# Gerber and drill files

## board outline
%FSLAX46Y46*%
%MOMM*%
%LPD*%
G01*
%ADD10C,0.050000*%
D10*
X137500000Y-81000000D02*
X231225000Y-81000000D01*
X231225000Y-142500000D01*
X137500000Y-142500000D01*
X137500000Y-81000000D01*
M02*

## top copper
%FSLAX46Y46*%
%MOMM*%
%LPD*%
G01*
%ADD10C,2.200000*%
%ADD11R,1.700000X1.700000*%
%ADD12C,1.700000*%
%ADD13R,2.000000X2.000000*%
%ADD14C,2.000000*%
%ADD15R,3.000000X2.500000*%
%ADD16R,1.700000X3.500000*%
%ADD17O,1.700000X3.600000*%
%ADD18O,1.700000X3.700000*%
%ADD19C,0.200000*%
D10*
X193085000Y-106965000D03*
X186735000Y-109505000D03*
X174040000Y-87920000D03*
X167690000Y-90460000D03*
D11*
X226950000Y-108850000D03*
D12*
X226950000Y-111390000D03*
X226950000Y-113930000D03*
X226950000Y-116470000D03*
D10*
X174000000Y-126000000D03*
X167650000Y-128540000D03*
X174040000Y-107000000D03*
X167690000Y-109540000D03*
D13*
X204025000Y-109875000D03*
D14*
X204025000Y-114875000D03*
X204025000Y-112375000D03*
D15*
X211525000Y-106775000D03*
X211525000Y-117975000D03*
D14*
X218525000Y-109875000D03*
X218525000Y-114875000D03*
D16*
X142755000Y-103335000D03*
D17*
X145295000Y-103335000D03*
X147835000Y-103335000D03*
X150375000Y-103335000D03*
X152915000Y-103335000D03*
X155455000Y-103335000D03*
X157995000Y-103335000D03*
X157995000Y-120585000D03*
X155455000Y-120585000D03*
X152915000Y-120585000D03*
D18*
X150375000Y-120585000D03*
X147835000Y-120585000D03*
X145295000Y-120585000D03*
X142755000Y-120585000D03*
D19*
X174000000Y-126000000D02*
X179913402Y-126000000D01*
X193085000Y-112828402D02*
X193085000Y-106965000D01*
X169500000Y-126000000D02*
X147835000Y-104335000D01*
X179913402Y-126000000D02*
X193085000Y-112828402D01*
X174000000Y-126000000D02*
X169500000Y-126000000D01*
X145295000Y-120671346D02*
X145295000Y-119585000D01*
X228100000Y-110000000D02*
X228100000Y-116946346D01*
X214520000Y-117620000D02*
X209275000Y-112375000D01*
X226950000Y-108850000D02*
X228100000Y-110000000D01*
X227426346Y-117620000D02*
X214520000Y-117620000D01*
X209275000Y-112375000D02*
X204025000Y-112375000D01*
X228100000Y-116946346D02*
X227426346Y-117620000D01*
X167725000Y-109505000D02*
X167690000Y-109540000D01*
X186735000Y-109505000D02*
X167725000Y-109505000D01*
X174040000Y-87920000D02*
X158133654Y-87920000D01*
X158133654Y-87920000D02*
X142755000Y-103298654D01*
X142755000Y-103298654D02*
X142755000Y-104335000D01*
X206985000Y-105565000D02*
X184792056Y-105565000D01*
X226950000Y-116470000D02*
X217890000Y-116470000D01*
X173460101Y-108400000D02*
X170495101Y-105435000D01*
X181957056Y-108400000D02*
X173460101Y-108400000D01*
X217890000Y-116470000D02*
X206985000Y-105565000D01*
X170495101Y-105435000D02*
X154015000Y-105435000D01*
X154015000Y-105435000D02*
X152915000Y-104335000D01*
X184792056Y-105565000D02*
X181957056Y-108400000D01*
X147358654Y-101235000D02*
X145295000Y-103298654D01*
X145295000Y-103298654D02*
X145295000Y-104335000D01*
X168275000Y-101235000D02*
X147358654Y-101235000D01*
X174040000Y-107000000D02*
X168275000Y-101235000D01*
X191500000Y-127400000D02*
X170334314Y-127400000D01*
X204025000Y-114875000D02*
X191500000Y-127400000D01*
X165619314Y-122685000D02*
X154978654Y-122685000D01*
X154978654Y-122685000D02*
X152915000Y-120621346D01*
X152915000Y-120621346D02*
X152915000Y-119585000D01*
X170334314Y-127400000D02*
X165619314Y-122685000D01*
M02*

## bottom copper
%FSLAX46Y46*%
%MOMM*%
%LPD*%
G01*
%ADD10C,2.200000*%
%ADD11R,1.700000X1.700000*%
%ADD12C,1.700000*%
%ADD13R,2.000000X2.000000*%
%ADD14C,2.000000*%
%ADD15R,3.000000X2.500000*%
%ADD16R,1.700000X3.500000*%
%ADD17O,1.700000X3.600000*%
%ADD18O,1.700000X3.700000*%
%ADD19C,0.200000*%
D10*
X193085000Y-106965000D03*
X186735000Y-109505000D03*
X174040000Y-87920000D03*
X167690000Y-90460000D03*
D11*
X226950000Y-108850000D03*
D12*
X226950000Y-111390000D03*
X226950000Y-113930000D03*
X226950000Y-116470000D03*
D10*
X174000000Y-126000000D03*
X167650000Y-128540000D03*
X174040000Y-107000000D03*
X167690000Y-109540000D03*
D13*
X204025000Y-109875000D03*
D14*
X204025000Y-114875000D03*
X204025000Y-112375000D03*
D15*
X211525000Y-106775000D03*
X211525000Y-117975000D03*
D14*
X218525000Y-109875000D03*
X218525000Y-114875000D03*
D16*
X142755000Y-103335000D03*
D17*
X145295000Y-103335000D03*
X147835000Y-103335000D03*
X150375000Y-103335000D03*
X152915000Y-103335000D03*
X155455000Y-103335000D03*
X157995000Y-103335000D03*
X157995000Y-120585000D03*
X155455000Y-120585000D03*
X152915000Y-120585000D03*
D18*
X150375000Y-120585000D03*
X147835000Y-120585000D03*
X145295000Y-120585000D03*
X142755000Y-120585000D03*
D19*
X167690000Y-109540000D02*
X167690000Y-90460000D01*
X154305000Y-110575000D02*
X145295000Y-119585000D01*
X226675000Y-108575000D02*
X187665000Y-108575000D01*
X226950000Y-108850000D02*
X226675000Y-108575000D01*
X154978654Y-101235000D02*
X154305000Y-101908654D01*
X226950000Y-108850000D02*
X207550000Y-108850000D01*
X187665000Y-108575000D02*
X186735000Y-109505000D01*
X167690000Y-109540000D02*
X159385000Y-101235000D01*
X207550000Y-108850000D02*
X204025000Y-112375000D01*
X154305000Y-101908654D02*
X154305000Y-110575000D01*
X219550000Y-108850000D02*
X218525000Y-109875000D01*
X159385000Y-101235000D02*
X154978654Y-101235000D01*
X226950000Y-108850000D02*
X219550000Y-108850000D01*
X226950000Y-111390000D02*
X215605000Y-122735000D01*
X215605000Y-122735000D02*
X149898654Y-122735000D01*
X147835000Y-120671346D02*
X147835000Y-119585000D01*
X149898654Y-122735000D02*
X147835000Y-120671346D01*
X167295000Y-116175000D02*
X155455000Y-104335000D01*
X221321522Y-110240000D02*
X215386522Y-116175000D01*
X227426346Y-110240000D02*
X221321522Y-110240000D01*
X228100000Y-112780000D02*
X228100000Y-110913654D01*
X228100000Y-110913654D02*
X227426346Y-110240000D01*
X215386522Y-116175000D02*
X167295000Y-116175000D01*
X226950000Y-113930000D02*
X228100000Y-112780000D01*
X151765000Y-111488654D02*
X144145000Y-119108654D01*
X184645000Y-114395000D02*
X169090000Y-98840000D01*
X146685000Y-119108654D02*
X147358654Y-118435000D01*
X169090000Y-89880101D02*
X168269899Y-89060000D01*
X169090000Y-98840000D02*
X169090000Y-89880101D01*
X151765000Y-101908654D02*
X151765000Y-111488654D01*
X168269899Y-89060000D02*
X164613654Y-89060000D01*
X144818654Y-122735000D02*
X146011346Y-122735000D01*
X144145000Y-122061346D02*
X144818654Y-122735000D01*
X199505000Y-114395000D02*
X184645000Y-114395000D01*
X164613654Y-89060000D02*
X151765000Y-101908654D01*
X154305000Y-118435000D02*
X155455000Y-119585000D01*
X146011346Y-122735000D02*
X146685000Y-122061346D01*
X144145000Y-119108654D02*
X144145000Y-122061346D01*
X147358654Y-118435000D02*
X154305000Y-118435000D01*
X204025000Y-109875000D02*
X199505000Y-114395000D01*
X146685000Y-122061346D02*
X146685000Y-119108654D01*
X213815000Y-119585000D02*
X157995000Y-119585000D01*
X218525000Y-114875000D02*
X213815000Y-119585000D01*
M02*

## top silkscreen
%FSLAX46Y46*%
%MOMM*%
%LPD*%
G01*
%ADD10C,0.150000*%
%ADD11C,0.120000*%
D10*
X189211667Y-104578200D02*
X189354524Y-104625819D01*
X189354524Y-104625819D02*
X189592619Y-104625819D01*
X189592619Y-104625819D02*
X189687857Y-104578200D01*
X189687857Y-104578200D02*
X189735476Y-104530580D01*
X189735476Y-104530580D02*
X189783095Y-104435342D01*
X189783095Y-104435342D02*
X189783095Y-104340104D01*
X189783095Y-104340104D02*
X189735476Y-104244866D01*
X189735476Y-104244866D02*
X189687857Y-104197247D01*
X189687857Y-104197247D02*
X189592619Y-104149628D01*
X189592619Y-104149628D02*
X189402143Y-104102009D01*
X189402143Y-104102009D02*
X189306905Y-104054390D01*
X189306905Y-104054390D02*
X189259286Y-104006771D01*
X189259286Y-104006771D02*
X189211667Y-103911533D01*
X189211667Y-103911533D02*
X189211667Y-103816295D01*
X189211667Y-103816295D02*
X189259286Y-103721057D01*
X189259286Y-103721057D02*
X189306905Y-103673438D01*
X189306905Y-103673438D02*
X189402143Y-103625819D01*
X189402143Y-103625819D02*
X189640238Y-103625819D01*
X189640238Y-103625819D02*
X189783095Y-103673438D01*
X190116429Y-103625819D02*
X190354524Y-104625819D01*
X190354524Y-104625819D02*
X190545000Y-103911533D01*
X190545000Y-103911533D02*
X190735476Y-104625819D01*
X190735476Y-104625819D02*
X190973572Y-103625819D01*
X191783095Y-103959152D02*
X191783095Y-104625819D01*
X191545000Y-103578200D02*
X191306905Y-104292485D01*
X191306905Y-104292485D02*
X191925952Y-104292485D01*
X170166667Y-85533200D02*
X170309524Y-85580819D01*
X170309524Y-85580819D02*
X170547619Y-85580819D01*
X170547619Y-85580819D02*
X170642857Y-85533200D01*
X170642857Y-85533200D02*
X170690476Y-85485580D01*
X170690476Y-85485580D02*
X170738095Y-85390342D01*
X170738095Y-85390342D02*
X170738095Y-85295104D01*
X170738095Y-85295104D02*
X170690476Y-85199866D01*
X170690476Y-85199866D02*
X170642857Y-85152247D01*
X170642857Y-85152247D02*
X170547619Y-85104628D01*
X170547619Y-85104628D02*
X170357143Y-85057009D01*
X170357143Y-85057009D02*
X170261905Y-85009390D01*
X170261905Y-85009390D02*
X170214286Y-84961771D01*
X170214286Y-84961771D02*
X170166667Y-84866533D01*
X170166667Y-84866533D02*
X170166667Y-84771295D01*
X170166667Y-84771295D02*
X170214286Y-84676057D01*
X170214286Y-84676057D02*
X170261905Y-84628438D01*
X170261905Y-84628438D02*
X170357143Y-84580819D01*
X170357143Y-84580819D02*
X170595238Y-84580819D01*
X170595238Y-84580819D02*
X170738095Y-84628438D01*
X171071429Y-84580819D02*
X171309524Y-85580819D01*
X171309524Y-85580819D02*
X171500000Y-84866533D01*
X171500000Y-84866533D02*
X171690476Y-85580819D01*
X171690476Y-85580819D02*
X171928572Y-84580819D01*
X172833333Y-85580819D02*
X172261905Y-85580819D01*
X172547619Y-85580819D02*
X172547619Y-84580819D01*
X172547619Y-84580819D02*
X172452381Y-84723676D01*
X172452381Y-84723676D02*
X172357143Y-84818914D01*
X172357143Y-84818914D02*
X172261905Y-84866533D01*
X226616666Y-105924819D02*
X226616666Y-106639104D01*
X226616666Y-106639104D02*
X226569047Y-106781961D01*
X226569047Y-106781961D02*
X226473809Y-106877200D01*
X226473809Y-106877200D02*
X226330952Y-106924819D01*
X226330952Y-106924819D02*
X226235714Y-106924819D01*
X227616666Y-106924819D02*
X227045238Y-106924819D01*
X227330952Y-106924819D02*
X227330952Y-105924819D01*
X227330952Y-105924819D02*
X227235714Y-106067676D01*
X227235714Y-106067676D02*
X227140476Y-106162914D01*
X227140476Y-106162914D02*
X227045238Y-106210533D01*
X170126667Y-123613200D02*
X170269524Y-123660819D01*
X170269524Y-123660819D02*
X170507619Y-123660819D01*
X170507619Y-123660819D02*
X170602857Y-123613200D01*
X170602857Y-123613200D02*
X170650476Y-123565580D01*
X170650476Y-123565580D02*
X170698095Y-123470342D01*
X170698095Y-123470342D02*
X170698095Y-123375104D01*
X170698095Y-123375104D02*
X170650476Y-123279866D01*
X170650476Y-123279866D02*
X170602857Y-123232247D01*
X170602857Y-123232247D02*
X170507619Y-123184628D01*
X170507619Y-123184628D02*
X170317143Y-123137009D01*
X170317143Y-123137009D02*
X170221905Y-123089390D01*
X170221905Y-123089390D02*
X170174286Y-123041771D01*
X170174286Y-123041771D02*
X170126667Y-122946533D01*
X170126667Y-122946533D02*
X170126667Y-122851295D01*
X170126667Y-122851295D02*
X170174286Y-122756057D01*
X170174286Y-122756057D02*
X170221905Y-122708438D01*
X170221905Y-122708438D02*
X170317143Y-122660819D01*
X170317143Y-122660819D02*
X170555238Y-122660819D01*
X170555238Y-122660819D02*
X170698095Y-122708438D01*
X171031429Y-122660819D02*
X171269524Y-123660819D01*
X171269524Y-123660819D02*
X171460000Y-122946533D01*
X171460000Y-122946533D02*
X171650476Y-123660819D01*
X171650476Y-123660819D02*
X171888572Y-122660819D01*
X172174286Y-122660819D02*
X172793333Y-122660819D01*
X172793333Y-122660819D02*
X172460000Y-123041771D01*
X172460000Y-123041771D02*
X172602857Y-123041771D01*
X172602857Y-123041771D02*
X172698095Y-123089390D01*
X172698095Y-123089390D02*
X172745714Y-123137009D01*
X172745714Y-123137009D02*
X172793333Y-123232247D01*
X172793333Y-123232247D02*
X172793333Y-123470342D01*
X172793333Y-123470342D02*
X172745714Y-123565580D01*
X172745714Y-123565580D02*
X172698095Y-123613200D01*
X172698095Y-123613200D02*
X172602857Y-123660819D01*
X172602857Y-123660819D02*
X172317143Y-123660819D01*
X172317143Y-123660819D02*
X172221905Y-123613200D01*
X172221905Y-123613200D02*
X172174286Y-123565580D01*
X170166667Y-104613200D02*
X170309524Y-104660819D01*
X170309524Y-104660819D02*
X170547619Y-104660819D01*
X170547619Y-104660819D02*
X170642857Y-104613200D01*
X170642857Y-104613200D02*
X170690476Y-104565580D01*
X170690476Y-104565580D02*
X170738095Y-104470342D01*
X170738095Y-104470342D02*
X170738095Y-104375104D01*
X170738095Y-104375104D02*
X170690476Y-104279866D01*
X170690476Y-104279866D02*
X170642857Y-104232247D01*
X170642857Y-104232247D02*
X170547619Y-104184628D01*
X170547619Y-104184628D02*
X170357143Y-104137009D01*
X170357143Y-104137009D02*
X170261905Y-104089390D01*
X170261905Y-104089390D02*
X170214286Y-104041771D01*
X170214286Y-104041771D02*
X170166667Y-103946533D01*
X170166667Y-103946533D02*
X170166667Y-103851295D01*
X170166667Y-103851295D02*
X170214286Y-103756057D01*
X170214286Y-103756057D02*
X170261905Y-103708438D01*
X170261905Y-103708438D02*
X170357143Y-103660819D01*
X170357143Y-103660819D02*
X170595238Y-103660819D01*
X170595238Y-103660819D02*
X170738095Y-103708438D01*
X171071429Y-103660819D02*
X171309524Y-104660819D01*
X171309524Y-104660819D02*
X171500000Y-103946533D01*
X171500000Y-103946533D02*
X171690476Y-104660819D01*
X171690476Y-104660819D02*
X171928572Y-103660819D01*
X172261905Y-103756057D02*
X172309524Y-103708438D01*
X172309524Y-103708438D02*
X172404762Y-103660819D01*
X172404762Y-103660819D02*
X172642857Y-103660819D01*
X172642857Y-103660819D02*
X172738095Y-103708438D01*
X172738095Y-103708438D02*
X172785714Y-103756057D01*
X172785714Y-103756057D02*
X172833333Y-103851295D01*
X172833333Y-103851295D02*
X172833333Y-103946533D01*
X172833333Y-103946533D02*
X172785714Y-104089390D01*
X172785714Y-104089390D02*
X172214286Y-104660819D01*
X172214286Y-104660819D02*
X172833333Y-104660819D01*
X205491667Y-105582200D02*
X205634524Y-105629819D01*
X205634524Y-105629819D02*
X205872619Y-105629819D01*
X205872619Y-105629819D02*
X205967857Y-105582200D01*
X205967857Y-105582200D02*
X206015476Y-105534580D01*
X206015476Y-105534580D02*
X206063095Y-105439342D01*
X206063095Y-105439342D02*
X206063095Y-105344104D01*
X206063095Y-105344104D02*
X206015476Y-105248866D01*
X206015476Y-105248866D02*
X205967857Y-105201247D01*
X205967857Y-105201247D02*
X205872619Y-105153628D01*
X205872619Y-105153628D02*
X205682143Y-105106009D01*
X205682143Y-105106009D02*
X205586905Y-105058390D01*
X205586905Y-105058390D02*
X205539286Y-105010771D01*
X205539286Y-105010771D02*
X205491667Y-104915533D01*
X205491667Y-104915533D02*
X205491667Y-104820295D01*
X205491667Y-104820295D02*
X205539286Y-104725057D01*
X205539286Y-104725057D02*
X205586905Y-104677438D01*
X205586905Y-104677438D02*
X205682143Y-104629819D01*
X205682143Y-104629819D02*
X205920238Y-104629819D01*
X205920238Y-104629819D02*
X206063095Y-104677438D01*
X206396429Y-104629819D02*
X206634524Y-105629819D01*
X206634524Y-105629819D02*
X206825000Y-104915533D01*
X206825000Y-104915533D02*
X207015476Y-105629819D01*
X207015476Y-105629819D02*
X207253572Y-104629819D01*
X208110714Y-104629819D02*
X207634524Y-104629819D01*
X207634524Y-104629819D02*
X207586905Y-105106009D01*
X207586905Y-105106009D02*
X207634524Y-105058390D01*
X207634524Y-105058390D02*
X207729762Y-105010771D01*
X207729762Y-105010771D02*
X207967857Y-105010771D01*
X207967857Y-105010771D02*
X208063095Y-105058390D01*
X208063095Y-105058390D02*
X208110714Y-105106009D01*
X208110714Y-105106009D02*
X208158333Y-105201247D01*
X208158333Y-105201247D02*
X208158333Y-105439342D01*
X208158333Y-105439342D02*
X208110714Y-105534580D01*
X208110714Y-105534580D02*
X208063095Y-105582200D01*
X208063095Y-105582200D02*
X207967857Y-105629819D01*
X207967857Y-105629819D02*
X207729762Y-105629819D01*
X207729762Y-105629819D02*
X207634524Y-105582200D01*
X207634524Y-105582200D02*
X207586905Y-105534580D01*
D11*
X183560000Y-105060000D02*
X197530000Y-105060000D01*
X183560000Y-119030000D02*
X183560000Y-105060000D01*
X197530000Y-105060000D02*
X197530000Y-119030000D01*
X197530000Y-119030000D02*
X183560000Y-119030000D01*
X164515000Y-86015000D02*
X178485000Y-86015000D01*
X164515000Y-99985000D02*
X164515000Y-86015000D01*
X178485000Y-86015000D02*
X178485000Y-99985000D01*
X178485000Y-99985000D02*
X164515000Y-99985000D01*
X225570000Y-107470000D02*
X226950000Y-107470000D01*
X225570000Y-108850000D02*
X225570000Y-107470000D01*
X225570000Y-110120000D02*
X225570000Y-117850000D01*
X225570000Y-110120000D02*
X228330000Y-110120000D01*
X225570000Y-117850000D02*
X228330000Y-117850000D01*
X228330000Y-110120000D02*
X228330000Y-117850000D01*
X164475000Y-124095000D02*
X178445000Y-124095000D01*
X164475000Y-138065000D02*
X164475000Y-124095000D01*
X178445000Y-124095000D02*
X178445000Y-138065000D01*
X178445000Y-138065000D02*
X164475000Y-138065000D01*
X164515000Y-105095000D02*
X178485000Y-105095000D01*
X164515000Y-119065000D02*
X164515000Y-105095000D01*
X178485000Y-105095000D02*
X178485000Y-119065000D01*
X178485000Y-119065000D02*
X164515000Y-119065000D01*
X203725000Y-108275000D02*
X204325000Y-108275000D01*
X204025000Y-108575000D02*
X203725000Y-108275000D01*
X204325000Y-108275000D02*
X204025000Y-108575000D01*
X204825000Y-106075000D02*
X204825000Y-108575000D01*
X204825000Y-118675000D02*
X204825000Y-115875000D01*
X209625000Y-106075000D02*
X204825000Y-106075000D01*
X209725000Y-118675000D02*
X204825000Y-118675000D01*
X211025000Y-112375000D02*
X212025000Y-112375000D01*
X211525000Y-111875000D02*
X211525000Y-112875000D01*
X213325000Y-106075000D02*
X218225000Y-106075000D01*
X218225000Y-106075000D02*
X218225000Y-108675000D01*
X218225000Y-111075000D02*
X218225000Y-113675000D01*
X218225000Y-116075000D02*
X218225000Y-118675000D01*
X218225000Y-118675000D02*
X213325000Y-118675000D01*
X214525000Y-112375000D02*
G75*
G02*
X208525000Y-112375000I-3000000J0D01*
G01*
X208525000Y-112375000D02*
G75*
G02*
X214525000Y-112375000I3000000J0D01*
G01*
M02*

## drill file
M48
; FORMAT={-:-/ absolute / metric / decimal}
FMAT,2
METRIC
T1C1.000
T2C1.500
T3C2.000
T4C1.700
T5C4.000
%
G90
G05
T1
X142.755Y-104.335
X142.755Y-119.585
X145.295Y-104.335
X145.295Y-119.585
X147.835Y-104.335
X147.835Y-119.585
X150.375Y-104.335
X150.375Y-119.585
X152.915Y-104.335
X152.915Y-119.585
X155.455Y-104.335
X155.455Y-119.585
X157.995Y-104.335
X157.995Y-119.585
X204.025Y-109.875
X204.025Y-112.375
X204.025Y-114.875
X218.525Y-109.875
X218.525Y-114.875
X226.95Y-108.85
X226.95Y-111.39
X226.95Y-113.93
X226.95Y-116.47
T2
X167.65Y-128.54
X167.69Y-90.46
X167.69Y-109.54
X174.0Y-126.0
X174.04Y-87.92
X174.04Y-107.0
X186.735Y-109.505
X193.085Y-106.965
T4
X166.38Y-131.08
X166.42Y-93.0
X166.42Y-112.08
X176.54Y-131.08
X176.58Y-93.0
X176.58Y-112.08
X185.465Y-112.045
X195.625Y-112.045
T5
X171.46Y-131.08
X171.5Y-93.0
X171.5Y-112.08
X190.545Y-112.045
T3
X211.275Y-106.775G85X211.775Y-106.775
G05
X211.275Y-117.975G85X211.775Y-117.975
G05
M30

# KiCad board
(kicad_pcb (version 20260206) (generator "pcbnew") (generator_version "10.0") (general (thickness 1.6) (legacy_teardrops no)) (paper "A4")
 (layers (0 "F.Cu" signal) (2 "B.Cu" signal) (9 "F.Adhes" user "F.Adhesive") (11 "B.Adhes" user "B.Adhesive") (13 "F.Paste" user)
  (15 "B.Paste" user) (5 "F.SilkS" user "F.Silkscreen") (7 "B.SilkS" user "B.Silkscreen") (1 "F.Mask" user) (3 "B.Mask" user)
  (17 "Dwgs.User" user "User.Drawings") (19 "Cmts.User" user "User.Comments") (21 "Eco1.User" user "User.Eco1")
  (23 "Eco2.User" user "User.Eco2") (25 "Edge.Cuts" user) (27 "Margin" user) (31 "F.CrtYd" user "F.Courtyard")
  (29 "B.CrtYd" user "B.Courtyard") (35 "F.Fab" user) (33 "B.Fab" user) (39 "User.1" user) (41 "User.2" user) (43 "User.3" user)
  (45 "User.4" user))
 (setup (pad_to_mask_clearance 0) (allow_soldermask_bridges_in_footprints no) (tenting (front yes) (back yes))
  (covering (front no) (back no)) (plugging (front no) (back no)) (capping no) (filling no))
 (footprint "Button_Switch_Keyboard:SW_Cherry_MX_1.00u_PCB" (layer "F.Cu") (at 193.085 106.965)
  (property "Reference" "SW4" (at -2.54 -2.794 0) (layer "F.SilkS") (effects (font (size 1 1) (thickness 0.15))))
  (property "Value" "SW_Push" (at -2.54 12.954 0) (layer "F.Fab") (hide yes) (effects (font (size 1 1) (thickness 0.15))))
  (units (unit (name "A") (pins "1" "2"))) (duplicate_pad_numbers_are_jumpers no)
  (fp_line (start -9.525 -1.905) (end 4.445 -1.905) (stroke (width 0.12) (type solid)) (layer "F.SilkS"))
  (fp_line (start -9.525 12.065) (end -9.525 -1.905) (stroke (width 0.12) (type solid)) (layer "F.SilkS"))
  (fp_line (start 4.445 -1.905) (end 4.445 12.065) (stroke (width 0.12) (type solid)) (layer "F.SilkS"))
  (fp_line (start 4.445 12.065) (end -9.525 12.065) (stroke (width 0.12) (type solid)) (layer "F.SilkS"))
  (pad "" np_thru_hole circle (at -7.62 5.08) (size 1.7 1.7) (drill 1.7) (layers "*.Cu" "*.Mask"))
  (pad "" np_thru_hole circle (at -2.54 5.08) (size 4 4) (drill 4) (layers "*.Cu" "*.Mask"))
  (pad "" np_thru_hole circle (at 2.54 5.08) (size 1.7 1.7) (drill 1.7) (layers "*.Cu" "*.Mask"))
  (pad "1" thru_hole circle (at 0 0) (size 2.2 2.2) (drill 1.5) (layers "*.Cu" "*.Mask") (remove_unused_layers no)
   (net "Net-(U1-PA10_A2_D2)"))
  (pad "2" thru_hole circle (at -6.35 2.54) (size 2.2 2.2) (drill 1.5) (layers "*.Cu" "*.Mask") (remove_unused_layers no) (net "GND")))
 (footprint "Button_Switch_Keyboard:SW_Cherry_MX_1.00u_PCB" (layer "F.Cu") (at 174.04 87.92)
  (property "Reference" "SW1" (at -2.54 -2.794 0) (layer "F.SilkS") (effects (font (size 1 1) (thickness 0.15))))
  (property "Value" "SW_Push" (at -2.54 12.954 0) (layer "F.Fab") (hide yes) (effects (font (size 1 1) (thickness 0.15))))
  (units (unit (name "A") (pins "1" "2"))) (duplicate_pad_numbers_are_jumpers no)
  (fp_line (start -9.525 -1.905) (end 4.445 -1.905) (stroke (width 0.12) (type solid)) (layer "F.SilkS"))
  (fp_line (start -9.525 12.065) (end -9.525 -1.905) (stroke (width 0.12) (type solid)) (layer "F.SilkS"))
  (fp_line (start 4.445 -1.905) (end 4.445 12.065) (stroke (width 0.12) (type solid)) (layer "F.SilkS"))
  (fp_line (start 4.445 12.065) (end -9.525 12.065) (stroke (width 0.12) (type solid)) (layer "F.SilkS"))
  (pad "" np_thru_hole circle (at -7.62 5.08) (size 1.7 1.7) (drill 1.7) (layers "*.Cu" "*.Mask"))
  (pad "" np_thru_hole circle (at -2.54 5.08) (size 4 4) (drill 4) (layers "*.Cu" "*.Mask"))
  (pad "" np_thru_hole circle (at 2.54 5.08) (size 1.7 1.7) (drill 1.7) (layers "*.Cu" "*.Mask"))
  (pad "1" thru_hole circle (at 0 0) (size 2.2 2.2) (drill 1.5) (layers "*.Cu" "*.Mask") (remove_unused_layers no)
   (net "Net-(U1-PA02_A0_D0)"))
  (pad "2" thru_hole circle (at -6.35 2.54) (size 2.2 2.2) (drill 1.5) (layers "*.Cu" "*.Mask") (remove_unused_layers no) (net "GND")))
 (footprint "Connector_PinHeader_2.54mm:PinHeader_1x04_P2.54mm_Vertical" (layer "F.Cu") (at 226.95 108.85)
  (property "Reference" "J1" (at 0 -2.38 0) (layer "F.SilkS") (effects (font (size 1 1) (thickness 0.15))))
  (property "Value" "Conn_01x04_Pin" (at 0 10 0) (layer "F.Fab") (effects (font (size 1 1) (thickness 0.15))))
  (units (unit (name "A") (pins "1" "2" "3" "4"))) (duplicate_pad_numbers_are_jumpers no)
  (fp_line (start -1.38 -1.38) (end 0 -1.38) (stroke (width 0.12) (type solid)) (layer "F.SilkS"))
  (fp_line (start -1.38 0) (end -1.38 -1.38) (stroke (width 0.12) (type solid)) (layer "F.SilkS"))
  (fp_line (start -1.38 1.27) (end -1.38 9) (stroke (width 0.12) (type solid)) (layer "F.SilkS"))
  (fp_line (start -1.38 1.27) (end 1.38 1.27) (stroke (width 0.12) (type solid)) (layer "F.SilkS"))
  (fp_line (start -1.38 9) (end 1.38 9) (stroke (width 0.12) (type solid)) (layer "F.SilkS"))
  (fp_line (start 1.38 1.27) (end 1.38 9) (stroke (width 0.12) (type solid)) (layer "F.SilkS"))
  (pad "1" thru_hole rect (at 0 0) (size 1.7 1.7) (drill 1) (layers "*.Cu" "*.Mask") (remove_unused_layers no) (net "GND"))
  (pad "2" thru_hole circle (at 0 2.54) (size 1.7 1.7) (drill 1) (layers "*.Cu" "*.Mask") (remove_unused_layers no) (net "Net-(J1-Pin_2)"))
  (pad "3" thru_hole circle (at 0 5.08) (size 1.7 1.7) (drill 1) (layers "*.Cu" "*.Mask") (remove_unused_layers no) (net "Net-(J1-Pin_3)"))
  (pad "4" thru_hole circle (at 0 7.62) (size 1.7 1.7) (drill 1) (layers "*.Cu" "*.Mask") (remove_unused_layers no) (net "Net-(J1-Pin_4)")))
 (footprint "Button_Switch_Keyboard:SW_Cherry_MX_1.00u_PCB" (layer "F.Cu") (at 174 126)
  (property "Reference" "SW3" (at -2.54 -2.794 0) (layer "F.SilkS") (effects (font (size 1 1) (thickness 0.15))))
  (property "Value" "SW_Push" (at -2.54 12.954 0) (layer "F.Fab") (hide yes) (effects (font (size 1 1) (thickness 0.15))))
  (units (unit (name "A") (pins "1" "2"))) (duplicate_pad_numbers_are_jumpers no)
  (fp_line (start -9.525 -1.905) (end 4.445 -1.905) (stroke (width 0.12) (type solid)) (layer "F.SilkS"))
  (fp_line (start -9.525 12.065) (end -9.525 -1.905) (stroke (width 0.12) (type solid)) (layer "F.SilkS"))
  (fp_line (start 4.445 -1.905) (end 4.445 12.065) (stroke (width 0.12) (type solid)) (layer "F.SilkS"))
  (fp_line (start 4.445 12.065) (end -9.525 12.065) (stroke (width 0.12) (type solid)) (layer "F.SilkS"))
  (pad "" np_thru_hole circle (at -7.62 5.08) (size 1.7 1.7) (drill 1.7) (layers "*.Cu" "*.Mask"))
  (pad "" np_thru_hole circle (at -2.54 5.08) (size 4 4) (drill 4) (layers "*.Cu" "*.Mask"))
  (pad "" np_thru_hole circle (at 2.54 5.08) (size 1.7 1.7) (drill 1.7) (layers "*.Cu" "*.Mask"))
  (pad "1" thru_hole circle (at 0 0) (size 2.2 2.2) (drill 1.5) (layers "*.Cu" "*.Mask") (remove_unused_layers no)
   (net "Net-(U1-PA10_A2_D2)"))
  (pad "2" thru_hole circle (at -6.35 2.54) (size 2.2 2.2) (drill 1.5) (layers "*.Cu" "*.Mask") (remove_unused_layers no) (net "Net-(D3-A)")))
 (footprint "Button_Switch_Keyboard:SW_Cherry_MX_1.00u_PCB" (layer "F.Cu") (at 174.04 107)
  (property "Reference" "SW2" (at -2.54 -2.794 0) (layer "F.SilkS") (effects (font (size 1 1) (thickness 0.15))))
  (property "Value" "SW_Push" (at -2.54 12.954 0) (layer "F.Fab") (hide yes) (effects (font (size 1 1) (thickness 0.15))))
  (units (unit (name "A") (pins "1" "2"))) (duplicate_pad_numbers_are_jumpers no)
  (fp_line (start -9.525 -1.905) (end 4.445 -1.905) (stroke (width 0.12) (type solid)) (layer "F.SilkS"))
  (fp_line (start -9.525 12.065) (end -9.525 -1.905) (stroke (width 0.12) (type solid)) (layer "F.SilkS"))
  (fp_line (start 4.445 -1.905) (end 4.445 12.065) (stroke (width 0.12) (type solid)) (layer "F.SilkS"))
  (fp_line (start 4.445 12.065) (end -9.525 12.065) (stroke (width 0.12) (type solid)) (layer "F.SilkS"))
  (pad "" np_thru_hole circle (at -7.62 5.08) (size 1.7 1.7) (drill 1.7) (layers "*.Cu" "*.Mask"))
  (pad "" np_thru_hole circle (at -2.54 5.08) (size 4 4) (drill 4) (layers "*.Cu" "*.Mask"))
  (pad "" np_thru_hole circle (at 2.54 5.08) (size 1.7 1.7) (drill 1.7) (layers "*.Cu" "*.Mask"))
  (pad "1" thru_hole circle (at 0 0) (size 2.2 2.2) (drill 1.5) (layers "*.Cu" "*.Mask") (remove_unused_layers no)
   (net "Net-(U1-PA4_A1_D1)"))
  (pad "2" thru_hole circle (at -6.35 2.54) (size 2.2 2.2) (drill 1.5) (layers "*.Cu" "*.Mask") (remove_unused_layers no) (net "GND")))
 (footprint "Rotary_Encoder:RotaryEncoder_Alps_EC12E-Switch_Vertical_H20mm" (layer "F.Cu") (at 204.025 109.875)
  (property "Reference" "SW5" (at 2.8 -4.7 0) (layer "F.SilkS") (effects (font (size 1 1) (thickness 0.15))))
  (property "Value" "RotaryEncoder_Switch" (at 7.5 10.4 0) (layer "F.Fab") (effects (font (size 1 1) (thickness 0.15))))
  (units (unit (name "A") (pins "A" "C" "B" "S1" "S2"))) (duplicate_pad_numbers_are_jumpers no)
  (fp_line (start -0.3 -1.6) (end 0.3 -1.6) (stroke (width 0.12) (type solid)) (layer "F.SilkS"))
  (fp_line (start 0 -1.3) (end -0.3 -1.6) (stroke (width 0.12) (type solid)) (layer "F.SilkS"))
  (fp_line (start 0.3 -1.6) (end 0 -1.3) (stroke (width 0.12) (type solid)) (layer "F.SilkS"))
  (fp_line (start 0.8 -3.8) (end 0.8 -1.3) (stroke (width 0.12) (type solid)) (layer "F.SilkS"))
  (fp_line (start 0.8 8.8) (end 0.8 6) (stroke (width 0.12) (type solid)) (layer "F.SilkS"))
  (fp_line (start 5.6 -3.8) (end 0.8 -3.8) (stroke (width 0.12) (type solid)) (layer "F.SilkS"))
  (fp_line (start 5.7 8.8) (end 0.8 8.8) (stroke (width 0.12) (type solid)) (layer "F.SilkS"))
  (fp_line (start 7 2.5) (end 8 2.5) (stroke (width 0.12) (type solid)) (layer "F.SilkS"))
  (fp_line (start 7.5 2) (end 7.5 3) (stroke (width 0.12) (type solid)) (layer "F.SilkS"))
  (fp_line (start 9.3 -3.8) (end 14.2 -3.8) (stroke (width 0.12) (type solid)) (layer "F.SilkS"))
  (fp_line (start 14.2 -3.8) (end 14.2 -1.2) (stroke (width 0.12) (type solid)) (layer "F.SilkS"))
  (fp_line (start 14.2 1.2) (end 14.2 3.8) (stroke (width 0.12) (type solid)) (layer "F.SilkS"))
  (fp_line (start 14.2 6.2) (end 14.2 8.8) (stroke (width 0.12) (type solid)) (layer "F.SilkS"))
  (fp_line (start 14.2 8.8) (end 9.3 8.8) (stroke (width 0.12) (type solid)) (layer "F.SilkS"))
  (fp_circle (center 7.5 2.5) (end 10.5 2.5) (stroke (width 0.12) (type solid)) (fill no) (layer "F.SilkS"))
  (pad "A" thru_hole rect (at 0 0) (size 2 2) (drill 1) (layers "*.Cu" "*.Mask") (remove_unused_layers no) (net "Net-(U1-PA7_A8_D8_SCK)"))
  (pad "B" thru_hole circle (at 0 5) (size 2 2) (drill 1) (layers "*.Cu" "*.Mask") (remove_unused_layers no) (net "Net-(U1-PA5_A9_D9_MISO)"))
  (pad "C" thru_hole circle (at 0 2.5) (size 2 2) (drill 1) (layers "*.Cu" "*.Mask") (remove_unused_layers no) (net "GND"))
  (pad "MP" thru_hole rect (at 7.5 -3.1) (size 3 2.5) (drill oval 2.5 2) (layers "*.Cu" "*.Mask") (remove_unused_layers no))
  (pad "MP" thru_hole rect (at 7.5 8.1) (size 3 2.5) (drill oval 2.5 2) (layers "*.Cu" "*.Mask") (remove_unused_layers no))
  (pad "S1" thru_hole circle (at 14.5 0) (size 2 2) (drill 1) (layers "*.Cu" "*.Mask") (remove_unused_layers no) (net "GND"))
  (pad "S2" thru_hole circle (at 14.5 5) (size 2 2) (drill 1) (layers "*.Cu" "*.Mask") (remove_unused_layers no)
   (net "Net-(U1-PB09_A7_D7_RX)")))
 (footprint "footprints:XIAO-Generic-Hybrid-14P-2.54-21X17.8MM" (layer "B.Cu") (at 150.375 111.96 -90)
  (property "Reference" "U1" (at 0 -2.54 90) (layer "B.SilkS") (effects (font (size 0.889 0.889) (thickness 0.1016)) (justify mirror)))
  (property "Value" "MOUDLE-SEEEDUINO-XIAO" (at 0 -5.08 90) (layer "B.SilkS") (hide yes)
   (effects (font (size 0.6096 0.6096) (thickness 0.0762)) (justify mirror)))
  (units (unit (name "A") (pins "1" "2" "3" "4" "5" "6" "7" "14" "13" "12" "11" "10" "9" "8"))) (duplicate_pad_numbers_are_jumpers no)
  (pad "1" thru_hole rect (at -7.625 7.62 270) (size 3.5 1.7) (drill 1 (offset -1 0)) (layers "*.Cu" "*.Mask") (remove_unused_layers no)
   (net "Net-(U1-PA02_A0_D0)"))
  (pad "2" thru_hole oval (at -7.625 5.08 270) (size 3.6 1.7) (drill 1 (offset -1 0)) (layers "*.Cu" "*.Mask") (remove_unused_layers no)
   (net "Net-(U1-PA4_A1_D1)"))
  (pad "3" thru_hole oval (at -7.625 2.54 270) (size 3.6 1.7) (drill 1 (offset -1 0)) (layers "*.Cu" "*.Mask") (remove_unused_layers no)
   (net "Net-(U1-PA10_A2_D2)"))
  (pad "4" thru_hole oval (at -7.625 0 270) (size 3.6 1.7) (drill 1 (offset -1 0)) (layers "*.Cu" "*.Mask") (remove_unused_layers no)
   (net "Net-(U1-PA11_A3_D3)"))
  (pad "5" thru_hole oval (at -7.625 -2.54 270) (size 3.6 1.7) (drill 1 (offset -1 0)) (layers "*.Cu" "*.Mask") (remove_unused_layers no)
   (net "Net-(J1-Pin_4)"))
  (pad "6" thru_hole oval (at -7.625 -5.08 90) (size 3.6 1.7) (drill 1 (offset 1 0)) (layers "*.Cu" "*.Mask") (remove_unused_layers no)
   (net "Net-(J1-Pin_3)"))
  (pad "7" thru_hole oval (at -7.625 -7.62 270) (size 3.6 1.7) (drill 1 (offset -1 0)) (layers "*.Cu" "*.Mask") (remove_unused_layers no)
   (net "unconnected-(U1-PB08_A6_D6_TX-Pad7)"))
  (pad "8" thru_hole oval (at 7.625 -7.62 270) (size 3.6 1.7) (drill 1 (offset 1 0)) (layers "*.Cu" "*.Mask") (remove_unused_layers no)
   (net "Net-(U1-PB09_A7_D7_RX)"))
  (pad "9" thru_hole oval (at 7.625 -5.08 270) (size 3.6 1.7) (drill 1 (offset 1 0)) (layers "*.Cu" "*.Mask") (remove_unused_layers no)
   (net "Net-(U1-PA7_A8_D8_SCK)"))
  (pad "10" thru_hole oval (at 7.625 -2.54 270) (size 3.6 1.7) (drill 1 (offset 1 0)) (layers "*.Cu" "*.Mask") (remove_unused_layers no)
   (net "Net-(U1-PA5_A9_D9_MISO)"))
  (pad "11" thru_hole oval (at 7.625 0 270) (size 3.7 1.7) (drill 1 (offset 1 0)) (layers "*.Cu" "*.Mask") (remove_unused_layers no)
   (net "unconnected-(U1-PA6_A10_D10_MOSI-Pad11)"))
  (pad "12" thru_hole oval (at 7.625 2.54 270) (size 3.7 1.7) (drill 1 (offset 1 0)) (layers "*.Cu" "*.Mask") (remove_unused_layers no)
   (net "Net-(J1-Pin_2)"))
  (pad "13" thru_hole oval (at 7.625 5.08 270) (size 3.7 1.7) (drill 1 (offset 1 0)) (layers "*.Cu" "*.Mask") (remove_unused_layers no)
   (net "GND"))
  (pad "14" thru_hole oval (at 7.625 7.62 270) (size 3.7 1.7) (drill 1 (offset 1 0)) (layers "*.Cu" "*.Mask") (remove_unused_layers no)
   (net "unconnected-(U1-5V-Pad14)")))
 (gr_rect (start 137.5 81) (end 231.225 142.5) (stroke (width 0.05) (type default)) (fill no) (layer "Edge.Cuts"))
 (segment (start 174 126) (end 179.913402 126) (width 0.2) (layer "F.Cu") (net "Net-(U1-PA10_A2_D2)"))
 (segment (start 193.085 112.828402) (end 193.085 106.965) (width 0.2) (layer "F.Cu") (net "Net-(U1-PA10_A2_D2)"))
 (segment (start 169.5 126) (end 147.835 104.335) (width 0.2) (layer "F.Cu") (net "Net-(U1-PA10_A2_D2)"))
 (segment (start 179.913402 126) (end 193.085 112.828402) (width 0.2) (layer "F.Cu") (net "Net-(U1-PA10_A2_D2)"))
 (segment (start 174 126) (end 169.5 126) (width 0.2) (layer "F.Cu") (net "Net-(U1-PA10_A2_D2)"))
 (segment (start 145.295 120.671346) (end 145.295 119.585) (width 0.2) (layer "F.Cu") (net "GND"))
 (segment (start 228.1 110) (end 228.1 116.946346) (width 0.2) (layer "F.Cu") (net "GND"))
 (segment (start 214.52 117.62) (end 209.275 112.375) (width 0.2) (layer "F.Cu") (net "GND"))
 (segment (start 226.95 108.85) (end 228.1 110) (width 0.2) (layer "F.Cu") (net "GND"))
 (segment (start 227.426346 117.62) (end 214.52 117.62) (width 0.2) (layer "F.Cu") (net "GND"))
 (segment (start 209.275 112.375) (end 204.025 112.375) (width 0.2) (layer "F.Cu") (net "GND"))
 (segment (start 228.1 116.946346) (end 227.426346 117.62) (width 0.2) (layer "F.Cu") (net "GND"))
 (segment (start 167.725 109.505) (end 167.69 109.54) (width 0.2) (layer "F.Cu") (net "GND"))
 (segment (start 186.735 109.505) (end 167.725 109.505) (width 0.2) (layer "F.Cu") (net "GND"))
 (segment (start 167.69 109.54) (end 167.69 90.46) (width 0.2) (layer "B.Cu") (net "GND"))
 (segment (start 154.305 110.575) (end 145.295 119.585) (width 0.2) (layer "B.Cu") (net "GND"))
 (segment (start 226.675 108.575) (end 187.665 108.575) (width 0.2) (layer "B.Cu") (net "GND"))
 (segment (start 226.95 108.85) (end 226.675 108.575) (width 0.2) (layer "B.Cu") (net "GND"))
 (segment (start 154.978654 101.235) (end 154.305 101.908654) (width 0.2) (layer "B.Cu") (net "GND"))
 (segment (start 226.95 108.85) (end 207.55 108.85) (width 0.2) (layer "B.Cu") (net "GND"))
 (segment (start 187.665 108.575) (end 186.735 109.505) (width 0.2) (layer "B.Cu") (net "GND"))
 (segment (start 167.69 109.54) (end 159.385 101.235) (width 0.2) (layer "B.Cu") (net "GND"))
 (segment (start 207.55 108.85) (end 204.025 112.375) (width 0.2) (layer "B.Cu") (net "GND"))
 (segment (start 154.305 101.908654) (end 154.305 110.575) (width 0.2) (layer "B.Cu") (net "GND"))
 (segment (start 219.55 108.85) (end 218.525 109.875) (width 0.2) (layer "B.Cu") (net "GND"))
 (segment (start 159.385 101.235) (end 154.978654 101.235) (width 0.2) (layer "B.Cu") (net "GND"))
 (segment (start 226.95 108.85) (end 219.55 108.85) (width 0.2) (layer "B.Cu") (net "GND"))
 (segment (start 174.04 87.92) (end 158.133654 87.92) (width 0.2) (layer "F.Cu") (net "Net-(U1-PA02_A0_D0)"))
 (segment (start 158.133654 87.92) (end 142.755 103.298654) (width 0.2) (layer "F.Cu") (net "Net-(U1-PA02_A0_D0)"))
 (segment (start 142.755 103.298654) (end 142.755 104.335) (width 0.2) (layer "F.Cu") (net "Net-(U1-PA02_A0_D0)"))
 (segment (start 226.95 111.39) (end 215.605 122.735) (width 0.2) (layer "B.Cu") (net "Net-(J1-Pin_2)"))
 (segment (start 215.605 122.735) (end 149.898654 122.735) (width 0.2) (layer "B.Cu") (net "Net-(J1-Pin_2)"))
 (segment (start 147.835 120.671346) (end 147.835 119.585) (width 0.2) (layer "B.Cu") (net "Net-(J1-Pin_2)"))
 (segment (start 149.898654 122.735) (end 147.835 120.671346) (width 0.2) (layer "B.Cu") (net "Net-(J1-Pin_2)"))
 (segment (start 167.295 116.175) (end 155.455 104.335) (width 0.2) (layer "B.Cu") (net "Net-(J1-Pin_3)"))
 (segment (start 221.321522 110.24) (end 215.386522 116.175) (width 0.2) (layer "B.Cu") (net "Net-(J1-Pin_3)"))
 (segment (start 227.426346 110.24) (end 221.321522 110.24) (width 0.2) (layer "B.Cu") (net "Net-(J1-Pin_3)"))
 (segment (start 228.1 112.78) (end 228.1 110.913654) (width 0.2) (layer "B.Cu") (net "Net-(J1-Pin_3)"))
 (segment (start 228.1 110.913654) (end 227.426346 110.24) (width 0.2) (layer "B.Cu") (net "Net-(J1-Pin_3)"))
 (segment (start 215.386522 116.175) (end 167.295 116.175) (width 0.2) (layer "B.Cu") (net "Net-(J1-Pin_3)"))
 (segment (start 226.95 113.93) (end 228.1 112.78) (width 0.2) (layer "B.Cu") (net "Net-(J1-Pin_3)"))
 (segment (start 206.985 105.565) (end 184.792056 105.565) (width 0.2) (layer "F.Cu") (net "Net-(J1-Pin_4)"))
 (segment (start 226.95 116.47) (end 217.89 116.47) (width 0.2) (layer "F.Cu") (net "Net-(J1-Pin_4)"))
 (segment (start 173.460101 108.4) (end 170.495101 105.435) (width 0.2) (layer "F.Cu") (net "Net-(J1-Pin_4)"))
 (segment (start 181.957056 108.4) (end 173.460101 108.4) (width 0.2) (layer "F.Cu") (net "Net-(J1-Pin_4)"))
 (segment (start 217.89 116.47) (end 206.985 105.565) (width 0.2) (layer "F.Cu") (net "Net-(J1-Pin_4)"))
 (segment (start 170.495101 105.435) (end 154.015 105.435) (width 0.2) (layer "F.Cu") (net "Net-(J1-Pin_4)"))
 (segment (start 154.015 105.435) (end 152.915 104.335) (width 0.2) (layer "F.Cu") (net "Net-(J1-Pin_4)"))
 (segment (start 184.792056 105.565) (end 181.957056 108.4) (width 0.2) (layer "F.Cu") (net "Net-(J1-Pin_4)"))
 (segment (start 147.358654 101.235) (end 145.295 103.298654) (width 0.2) (layer "F.Cu") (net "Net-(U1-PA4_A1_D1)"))
 (segment (start 145.295 103.298654) (end 145.295 104.335) (width 0.2) (layer "F.Cu") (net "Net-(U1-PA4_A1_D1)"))
 (segment (start 168.275 101.235) (end 147.358654 101.235) (width 0.2) (layer "F.Cu") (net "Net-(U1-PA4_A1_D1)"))
 (segment (start 174.04 107) (end 168.275 101.235) (width 0.2) (layer "F.Cu") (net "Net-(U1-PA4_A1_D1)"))
 (segment (start 151.765 111.488654) (end 144.145 119.108654) (width 0.2) (layer "B.Cu") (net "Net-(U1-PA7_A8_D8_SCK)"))
 (segment (start 184.645 114.395) (end 169.09 98.84) (width 0.2) (layer "B.Cu") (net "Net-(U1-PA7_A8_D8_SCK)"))
 (segment (start 146.685 119.108654) (end 147.358654 118.435) (width 0.2) (layer "B.Cu") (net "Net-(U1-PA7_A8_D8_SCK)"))
 (segment (start 169.09 89.880101) (end 168.269899 89.06) (width 0.2) (layer "B.Cu") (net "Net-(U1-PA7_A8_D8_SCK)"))
 (segment (start 169.09 98.84) (end 169.09 89.880101) (width 0.2) (layer "B.Cu") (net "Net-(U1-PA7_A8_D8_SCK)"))
 (segment (start 151.765 101.908654) (end 151.765 111.488654) (width 0.2) (layer "B.Cu") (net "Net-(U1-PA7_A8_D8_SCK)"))
 (segment (start 168.269899 89.06) (end 164.613654 89.06) (width 0.2) (layer "B.Cu") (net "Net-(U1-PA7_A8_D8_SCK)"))
 (segment (start 144.818654 122.735) (end 146.011346 122.735) (width 0.2) (layer "B.Cu") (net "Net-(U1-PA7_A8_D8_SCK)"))
 (segment (start 144.145 122.061346) (end 144.818654 122.735) (width 0.2) (layer "B.Cu") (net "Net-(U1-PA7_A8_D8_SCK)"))
 (segment (start 199.505 114.395) (end 184.645 114.395) (width 0.2) (layer "B.Cu") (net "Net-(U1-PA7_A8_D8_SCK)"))
 (segment (start 164.613654 89.06) (end 151.765 101.908654) (width 0.2) (layer "B.Cu") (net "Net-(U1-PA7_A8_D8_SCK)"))
 (segment (start 154.305 118.435) (end 155.455 119.585) (width 0.2) (layer "B.Cu") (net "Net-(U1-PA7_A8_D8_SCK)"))
 (segment (start 146.011346 122.735) (end 146.685 122.061346) (width 0.2) (layer "B.Cu") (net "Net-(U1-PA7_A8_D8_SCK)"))
 (segment (start 144.145 119.108654) (end 144.145 122.061346) (width 0.2) (layer "B.Cu") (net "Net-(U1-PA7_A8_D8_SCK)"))
 (segment (start 147.358654 118.435) (end 154.305 118.435) (width 0.2) (layer "B.Cu") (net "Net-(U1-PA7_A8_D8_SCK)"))
 (segment (start 204.025 109.875) (end 199.505 114.395) (width 0.2) (layer "B.Cu") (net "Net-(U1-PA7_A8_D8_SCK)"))
 (segment (start 146.685 122.061346) (end 146.685 119.108654) (width 0.2) (layer "B.Cu") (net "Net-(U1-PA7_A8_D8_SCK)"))
 (segment (start 191.5 127.4) (end 170.334314 127.4) (width 0.2) (layer "F.Cu") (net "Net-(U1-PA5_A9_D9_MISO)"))
 (segment (start 204.025 114.875) (end 191.5 127.4) (width 0.2) (layer "F.Cu") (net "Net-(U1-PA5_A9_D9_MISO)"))
 (segment (start 165.619314 122.685) (end 154.978654 122.685) (width 0.2) (layer "F.Cu") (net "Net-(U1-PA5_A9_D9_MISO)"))
 (segment (start 154.978654 122.685) (end 152.915 120.621346) (width 0.2) (layer "F.Cu") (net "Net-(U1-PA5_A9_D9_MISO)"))
 (segment (start 152.915 120.621346) (end 152.915 119.585) (width 0.2) (layer "F.Cu") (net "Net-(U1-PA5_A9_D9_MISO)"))
 (segment (start 170.334314 127.4) (end 165.619314 122.685) (width 0.2) (layer "F.Cu") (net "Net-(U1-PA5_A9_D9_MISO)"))
 (segment (start 213.815 119.585) (end 157.995 119.585) (width 0.2) (layer "B.Cu") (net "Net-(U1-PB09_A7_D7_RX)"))
 (segment (start 218.525 114.875) (end 213.815 119.585) (width 0.2) (layer "B.Cu") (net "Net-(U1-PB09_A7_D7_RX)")))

